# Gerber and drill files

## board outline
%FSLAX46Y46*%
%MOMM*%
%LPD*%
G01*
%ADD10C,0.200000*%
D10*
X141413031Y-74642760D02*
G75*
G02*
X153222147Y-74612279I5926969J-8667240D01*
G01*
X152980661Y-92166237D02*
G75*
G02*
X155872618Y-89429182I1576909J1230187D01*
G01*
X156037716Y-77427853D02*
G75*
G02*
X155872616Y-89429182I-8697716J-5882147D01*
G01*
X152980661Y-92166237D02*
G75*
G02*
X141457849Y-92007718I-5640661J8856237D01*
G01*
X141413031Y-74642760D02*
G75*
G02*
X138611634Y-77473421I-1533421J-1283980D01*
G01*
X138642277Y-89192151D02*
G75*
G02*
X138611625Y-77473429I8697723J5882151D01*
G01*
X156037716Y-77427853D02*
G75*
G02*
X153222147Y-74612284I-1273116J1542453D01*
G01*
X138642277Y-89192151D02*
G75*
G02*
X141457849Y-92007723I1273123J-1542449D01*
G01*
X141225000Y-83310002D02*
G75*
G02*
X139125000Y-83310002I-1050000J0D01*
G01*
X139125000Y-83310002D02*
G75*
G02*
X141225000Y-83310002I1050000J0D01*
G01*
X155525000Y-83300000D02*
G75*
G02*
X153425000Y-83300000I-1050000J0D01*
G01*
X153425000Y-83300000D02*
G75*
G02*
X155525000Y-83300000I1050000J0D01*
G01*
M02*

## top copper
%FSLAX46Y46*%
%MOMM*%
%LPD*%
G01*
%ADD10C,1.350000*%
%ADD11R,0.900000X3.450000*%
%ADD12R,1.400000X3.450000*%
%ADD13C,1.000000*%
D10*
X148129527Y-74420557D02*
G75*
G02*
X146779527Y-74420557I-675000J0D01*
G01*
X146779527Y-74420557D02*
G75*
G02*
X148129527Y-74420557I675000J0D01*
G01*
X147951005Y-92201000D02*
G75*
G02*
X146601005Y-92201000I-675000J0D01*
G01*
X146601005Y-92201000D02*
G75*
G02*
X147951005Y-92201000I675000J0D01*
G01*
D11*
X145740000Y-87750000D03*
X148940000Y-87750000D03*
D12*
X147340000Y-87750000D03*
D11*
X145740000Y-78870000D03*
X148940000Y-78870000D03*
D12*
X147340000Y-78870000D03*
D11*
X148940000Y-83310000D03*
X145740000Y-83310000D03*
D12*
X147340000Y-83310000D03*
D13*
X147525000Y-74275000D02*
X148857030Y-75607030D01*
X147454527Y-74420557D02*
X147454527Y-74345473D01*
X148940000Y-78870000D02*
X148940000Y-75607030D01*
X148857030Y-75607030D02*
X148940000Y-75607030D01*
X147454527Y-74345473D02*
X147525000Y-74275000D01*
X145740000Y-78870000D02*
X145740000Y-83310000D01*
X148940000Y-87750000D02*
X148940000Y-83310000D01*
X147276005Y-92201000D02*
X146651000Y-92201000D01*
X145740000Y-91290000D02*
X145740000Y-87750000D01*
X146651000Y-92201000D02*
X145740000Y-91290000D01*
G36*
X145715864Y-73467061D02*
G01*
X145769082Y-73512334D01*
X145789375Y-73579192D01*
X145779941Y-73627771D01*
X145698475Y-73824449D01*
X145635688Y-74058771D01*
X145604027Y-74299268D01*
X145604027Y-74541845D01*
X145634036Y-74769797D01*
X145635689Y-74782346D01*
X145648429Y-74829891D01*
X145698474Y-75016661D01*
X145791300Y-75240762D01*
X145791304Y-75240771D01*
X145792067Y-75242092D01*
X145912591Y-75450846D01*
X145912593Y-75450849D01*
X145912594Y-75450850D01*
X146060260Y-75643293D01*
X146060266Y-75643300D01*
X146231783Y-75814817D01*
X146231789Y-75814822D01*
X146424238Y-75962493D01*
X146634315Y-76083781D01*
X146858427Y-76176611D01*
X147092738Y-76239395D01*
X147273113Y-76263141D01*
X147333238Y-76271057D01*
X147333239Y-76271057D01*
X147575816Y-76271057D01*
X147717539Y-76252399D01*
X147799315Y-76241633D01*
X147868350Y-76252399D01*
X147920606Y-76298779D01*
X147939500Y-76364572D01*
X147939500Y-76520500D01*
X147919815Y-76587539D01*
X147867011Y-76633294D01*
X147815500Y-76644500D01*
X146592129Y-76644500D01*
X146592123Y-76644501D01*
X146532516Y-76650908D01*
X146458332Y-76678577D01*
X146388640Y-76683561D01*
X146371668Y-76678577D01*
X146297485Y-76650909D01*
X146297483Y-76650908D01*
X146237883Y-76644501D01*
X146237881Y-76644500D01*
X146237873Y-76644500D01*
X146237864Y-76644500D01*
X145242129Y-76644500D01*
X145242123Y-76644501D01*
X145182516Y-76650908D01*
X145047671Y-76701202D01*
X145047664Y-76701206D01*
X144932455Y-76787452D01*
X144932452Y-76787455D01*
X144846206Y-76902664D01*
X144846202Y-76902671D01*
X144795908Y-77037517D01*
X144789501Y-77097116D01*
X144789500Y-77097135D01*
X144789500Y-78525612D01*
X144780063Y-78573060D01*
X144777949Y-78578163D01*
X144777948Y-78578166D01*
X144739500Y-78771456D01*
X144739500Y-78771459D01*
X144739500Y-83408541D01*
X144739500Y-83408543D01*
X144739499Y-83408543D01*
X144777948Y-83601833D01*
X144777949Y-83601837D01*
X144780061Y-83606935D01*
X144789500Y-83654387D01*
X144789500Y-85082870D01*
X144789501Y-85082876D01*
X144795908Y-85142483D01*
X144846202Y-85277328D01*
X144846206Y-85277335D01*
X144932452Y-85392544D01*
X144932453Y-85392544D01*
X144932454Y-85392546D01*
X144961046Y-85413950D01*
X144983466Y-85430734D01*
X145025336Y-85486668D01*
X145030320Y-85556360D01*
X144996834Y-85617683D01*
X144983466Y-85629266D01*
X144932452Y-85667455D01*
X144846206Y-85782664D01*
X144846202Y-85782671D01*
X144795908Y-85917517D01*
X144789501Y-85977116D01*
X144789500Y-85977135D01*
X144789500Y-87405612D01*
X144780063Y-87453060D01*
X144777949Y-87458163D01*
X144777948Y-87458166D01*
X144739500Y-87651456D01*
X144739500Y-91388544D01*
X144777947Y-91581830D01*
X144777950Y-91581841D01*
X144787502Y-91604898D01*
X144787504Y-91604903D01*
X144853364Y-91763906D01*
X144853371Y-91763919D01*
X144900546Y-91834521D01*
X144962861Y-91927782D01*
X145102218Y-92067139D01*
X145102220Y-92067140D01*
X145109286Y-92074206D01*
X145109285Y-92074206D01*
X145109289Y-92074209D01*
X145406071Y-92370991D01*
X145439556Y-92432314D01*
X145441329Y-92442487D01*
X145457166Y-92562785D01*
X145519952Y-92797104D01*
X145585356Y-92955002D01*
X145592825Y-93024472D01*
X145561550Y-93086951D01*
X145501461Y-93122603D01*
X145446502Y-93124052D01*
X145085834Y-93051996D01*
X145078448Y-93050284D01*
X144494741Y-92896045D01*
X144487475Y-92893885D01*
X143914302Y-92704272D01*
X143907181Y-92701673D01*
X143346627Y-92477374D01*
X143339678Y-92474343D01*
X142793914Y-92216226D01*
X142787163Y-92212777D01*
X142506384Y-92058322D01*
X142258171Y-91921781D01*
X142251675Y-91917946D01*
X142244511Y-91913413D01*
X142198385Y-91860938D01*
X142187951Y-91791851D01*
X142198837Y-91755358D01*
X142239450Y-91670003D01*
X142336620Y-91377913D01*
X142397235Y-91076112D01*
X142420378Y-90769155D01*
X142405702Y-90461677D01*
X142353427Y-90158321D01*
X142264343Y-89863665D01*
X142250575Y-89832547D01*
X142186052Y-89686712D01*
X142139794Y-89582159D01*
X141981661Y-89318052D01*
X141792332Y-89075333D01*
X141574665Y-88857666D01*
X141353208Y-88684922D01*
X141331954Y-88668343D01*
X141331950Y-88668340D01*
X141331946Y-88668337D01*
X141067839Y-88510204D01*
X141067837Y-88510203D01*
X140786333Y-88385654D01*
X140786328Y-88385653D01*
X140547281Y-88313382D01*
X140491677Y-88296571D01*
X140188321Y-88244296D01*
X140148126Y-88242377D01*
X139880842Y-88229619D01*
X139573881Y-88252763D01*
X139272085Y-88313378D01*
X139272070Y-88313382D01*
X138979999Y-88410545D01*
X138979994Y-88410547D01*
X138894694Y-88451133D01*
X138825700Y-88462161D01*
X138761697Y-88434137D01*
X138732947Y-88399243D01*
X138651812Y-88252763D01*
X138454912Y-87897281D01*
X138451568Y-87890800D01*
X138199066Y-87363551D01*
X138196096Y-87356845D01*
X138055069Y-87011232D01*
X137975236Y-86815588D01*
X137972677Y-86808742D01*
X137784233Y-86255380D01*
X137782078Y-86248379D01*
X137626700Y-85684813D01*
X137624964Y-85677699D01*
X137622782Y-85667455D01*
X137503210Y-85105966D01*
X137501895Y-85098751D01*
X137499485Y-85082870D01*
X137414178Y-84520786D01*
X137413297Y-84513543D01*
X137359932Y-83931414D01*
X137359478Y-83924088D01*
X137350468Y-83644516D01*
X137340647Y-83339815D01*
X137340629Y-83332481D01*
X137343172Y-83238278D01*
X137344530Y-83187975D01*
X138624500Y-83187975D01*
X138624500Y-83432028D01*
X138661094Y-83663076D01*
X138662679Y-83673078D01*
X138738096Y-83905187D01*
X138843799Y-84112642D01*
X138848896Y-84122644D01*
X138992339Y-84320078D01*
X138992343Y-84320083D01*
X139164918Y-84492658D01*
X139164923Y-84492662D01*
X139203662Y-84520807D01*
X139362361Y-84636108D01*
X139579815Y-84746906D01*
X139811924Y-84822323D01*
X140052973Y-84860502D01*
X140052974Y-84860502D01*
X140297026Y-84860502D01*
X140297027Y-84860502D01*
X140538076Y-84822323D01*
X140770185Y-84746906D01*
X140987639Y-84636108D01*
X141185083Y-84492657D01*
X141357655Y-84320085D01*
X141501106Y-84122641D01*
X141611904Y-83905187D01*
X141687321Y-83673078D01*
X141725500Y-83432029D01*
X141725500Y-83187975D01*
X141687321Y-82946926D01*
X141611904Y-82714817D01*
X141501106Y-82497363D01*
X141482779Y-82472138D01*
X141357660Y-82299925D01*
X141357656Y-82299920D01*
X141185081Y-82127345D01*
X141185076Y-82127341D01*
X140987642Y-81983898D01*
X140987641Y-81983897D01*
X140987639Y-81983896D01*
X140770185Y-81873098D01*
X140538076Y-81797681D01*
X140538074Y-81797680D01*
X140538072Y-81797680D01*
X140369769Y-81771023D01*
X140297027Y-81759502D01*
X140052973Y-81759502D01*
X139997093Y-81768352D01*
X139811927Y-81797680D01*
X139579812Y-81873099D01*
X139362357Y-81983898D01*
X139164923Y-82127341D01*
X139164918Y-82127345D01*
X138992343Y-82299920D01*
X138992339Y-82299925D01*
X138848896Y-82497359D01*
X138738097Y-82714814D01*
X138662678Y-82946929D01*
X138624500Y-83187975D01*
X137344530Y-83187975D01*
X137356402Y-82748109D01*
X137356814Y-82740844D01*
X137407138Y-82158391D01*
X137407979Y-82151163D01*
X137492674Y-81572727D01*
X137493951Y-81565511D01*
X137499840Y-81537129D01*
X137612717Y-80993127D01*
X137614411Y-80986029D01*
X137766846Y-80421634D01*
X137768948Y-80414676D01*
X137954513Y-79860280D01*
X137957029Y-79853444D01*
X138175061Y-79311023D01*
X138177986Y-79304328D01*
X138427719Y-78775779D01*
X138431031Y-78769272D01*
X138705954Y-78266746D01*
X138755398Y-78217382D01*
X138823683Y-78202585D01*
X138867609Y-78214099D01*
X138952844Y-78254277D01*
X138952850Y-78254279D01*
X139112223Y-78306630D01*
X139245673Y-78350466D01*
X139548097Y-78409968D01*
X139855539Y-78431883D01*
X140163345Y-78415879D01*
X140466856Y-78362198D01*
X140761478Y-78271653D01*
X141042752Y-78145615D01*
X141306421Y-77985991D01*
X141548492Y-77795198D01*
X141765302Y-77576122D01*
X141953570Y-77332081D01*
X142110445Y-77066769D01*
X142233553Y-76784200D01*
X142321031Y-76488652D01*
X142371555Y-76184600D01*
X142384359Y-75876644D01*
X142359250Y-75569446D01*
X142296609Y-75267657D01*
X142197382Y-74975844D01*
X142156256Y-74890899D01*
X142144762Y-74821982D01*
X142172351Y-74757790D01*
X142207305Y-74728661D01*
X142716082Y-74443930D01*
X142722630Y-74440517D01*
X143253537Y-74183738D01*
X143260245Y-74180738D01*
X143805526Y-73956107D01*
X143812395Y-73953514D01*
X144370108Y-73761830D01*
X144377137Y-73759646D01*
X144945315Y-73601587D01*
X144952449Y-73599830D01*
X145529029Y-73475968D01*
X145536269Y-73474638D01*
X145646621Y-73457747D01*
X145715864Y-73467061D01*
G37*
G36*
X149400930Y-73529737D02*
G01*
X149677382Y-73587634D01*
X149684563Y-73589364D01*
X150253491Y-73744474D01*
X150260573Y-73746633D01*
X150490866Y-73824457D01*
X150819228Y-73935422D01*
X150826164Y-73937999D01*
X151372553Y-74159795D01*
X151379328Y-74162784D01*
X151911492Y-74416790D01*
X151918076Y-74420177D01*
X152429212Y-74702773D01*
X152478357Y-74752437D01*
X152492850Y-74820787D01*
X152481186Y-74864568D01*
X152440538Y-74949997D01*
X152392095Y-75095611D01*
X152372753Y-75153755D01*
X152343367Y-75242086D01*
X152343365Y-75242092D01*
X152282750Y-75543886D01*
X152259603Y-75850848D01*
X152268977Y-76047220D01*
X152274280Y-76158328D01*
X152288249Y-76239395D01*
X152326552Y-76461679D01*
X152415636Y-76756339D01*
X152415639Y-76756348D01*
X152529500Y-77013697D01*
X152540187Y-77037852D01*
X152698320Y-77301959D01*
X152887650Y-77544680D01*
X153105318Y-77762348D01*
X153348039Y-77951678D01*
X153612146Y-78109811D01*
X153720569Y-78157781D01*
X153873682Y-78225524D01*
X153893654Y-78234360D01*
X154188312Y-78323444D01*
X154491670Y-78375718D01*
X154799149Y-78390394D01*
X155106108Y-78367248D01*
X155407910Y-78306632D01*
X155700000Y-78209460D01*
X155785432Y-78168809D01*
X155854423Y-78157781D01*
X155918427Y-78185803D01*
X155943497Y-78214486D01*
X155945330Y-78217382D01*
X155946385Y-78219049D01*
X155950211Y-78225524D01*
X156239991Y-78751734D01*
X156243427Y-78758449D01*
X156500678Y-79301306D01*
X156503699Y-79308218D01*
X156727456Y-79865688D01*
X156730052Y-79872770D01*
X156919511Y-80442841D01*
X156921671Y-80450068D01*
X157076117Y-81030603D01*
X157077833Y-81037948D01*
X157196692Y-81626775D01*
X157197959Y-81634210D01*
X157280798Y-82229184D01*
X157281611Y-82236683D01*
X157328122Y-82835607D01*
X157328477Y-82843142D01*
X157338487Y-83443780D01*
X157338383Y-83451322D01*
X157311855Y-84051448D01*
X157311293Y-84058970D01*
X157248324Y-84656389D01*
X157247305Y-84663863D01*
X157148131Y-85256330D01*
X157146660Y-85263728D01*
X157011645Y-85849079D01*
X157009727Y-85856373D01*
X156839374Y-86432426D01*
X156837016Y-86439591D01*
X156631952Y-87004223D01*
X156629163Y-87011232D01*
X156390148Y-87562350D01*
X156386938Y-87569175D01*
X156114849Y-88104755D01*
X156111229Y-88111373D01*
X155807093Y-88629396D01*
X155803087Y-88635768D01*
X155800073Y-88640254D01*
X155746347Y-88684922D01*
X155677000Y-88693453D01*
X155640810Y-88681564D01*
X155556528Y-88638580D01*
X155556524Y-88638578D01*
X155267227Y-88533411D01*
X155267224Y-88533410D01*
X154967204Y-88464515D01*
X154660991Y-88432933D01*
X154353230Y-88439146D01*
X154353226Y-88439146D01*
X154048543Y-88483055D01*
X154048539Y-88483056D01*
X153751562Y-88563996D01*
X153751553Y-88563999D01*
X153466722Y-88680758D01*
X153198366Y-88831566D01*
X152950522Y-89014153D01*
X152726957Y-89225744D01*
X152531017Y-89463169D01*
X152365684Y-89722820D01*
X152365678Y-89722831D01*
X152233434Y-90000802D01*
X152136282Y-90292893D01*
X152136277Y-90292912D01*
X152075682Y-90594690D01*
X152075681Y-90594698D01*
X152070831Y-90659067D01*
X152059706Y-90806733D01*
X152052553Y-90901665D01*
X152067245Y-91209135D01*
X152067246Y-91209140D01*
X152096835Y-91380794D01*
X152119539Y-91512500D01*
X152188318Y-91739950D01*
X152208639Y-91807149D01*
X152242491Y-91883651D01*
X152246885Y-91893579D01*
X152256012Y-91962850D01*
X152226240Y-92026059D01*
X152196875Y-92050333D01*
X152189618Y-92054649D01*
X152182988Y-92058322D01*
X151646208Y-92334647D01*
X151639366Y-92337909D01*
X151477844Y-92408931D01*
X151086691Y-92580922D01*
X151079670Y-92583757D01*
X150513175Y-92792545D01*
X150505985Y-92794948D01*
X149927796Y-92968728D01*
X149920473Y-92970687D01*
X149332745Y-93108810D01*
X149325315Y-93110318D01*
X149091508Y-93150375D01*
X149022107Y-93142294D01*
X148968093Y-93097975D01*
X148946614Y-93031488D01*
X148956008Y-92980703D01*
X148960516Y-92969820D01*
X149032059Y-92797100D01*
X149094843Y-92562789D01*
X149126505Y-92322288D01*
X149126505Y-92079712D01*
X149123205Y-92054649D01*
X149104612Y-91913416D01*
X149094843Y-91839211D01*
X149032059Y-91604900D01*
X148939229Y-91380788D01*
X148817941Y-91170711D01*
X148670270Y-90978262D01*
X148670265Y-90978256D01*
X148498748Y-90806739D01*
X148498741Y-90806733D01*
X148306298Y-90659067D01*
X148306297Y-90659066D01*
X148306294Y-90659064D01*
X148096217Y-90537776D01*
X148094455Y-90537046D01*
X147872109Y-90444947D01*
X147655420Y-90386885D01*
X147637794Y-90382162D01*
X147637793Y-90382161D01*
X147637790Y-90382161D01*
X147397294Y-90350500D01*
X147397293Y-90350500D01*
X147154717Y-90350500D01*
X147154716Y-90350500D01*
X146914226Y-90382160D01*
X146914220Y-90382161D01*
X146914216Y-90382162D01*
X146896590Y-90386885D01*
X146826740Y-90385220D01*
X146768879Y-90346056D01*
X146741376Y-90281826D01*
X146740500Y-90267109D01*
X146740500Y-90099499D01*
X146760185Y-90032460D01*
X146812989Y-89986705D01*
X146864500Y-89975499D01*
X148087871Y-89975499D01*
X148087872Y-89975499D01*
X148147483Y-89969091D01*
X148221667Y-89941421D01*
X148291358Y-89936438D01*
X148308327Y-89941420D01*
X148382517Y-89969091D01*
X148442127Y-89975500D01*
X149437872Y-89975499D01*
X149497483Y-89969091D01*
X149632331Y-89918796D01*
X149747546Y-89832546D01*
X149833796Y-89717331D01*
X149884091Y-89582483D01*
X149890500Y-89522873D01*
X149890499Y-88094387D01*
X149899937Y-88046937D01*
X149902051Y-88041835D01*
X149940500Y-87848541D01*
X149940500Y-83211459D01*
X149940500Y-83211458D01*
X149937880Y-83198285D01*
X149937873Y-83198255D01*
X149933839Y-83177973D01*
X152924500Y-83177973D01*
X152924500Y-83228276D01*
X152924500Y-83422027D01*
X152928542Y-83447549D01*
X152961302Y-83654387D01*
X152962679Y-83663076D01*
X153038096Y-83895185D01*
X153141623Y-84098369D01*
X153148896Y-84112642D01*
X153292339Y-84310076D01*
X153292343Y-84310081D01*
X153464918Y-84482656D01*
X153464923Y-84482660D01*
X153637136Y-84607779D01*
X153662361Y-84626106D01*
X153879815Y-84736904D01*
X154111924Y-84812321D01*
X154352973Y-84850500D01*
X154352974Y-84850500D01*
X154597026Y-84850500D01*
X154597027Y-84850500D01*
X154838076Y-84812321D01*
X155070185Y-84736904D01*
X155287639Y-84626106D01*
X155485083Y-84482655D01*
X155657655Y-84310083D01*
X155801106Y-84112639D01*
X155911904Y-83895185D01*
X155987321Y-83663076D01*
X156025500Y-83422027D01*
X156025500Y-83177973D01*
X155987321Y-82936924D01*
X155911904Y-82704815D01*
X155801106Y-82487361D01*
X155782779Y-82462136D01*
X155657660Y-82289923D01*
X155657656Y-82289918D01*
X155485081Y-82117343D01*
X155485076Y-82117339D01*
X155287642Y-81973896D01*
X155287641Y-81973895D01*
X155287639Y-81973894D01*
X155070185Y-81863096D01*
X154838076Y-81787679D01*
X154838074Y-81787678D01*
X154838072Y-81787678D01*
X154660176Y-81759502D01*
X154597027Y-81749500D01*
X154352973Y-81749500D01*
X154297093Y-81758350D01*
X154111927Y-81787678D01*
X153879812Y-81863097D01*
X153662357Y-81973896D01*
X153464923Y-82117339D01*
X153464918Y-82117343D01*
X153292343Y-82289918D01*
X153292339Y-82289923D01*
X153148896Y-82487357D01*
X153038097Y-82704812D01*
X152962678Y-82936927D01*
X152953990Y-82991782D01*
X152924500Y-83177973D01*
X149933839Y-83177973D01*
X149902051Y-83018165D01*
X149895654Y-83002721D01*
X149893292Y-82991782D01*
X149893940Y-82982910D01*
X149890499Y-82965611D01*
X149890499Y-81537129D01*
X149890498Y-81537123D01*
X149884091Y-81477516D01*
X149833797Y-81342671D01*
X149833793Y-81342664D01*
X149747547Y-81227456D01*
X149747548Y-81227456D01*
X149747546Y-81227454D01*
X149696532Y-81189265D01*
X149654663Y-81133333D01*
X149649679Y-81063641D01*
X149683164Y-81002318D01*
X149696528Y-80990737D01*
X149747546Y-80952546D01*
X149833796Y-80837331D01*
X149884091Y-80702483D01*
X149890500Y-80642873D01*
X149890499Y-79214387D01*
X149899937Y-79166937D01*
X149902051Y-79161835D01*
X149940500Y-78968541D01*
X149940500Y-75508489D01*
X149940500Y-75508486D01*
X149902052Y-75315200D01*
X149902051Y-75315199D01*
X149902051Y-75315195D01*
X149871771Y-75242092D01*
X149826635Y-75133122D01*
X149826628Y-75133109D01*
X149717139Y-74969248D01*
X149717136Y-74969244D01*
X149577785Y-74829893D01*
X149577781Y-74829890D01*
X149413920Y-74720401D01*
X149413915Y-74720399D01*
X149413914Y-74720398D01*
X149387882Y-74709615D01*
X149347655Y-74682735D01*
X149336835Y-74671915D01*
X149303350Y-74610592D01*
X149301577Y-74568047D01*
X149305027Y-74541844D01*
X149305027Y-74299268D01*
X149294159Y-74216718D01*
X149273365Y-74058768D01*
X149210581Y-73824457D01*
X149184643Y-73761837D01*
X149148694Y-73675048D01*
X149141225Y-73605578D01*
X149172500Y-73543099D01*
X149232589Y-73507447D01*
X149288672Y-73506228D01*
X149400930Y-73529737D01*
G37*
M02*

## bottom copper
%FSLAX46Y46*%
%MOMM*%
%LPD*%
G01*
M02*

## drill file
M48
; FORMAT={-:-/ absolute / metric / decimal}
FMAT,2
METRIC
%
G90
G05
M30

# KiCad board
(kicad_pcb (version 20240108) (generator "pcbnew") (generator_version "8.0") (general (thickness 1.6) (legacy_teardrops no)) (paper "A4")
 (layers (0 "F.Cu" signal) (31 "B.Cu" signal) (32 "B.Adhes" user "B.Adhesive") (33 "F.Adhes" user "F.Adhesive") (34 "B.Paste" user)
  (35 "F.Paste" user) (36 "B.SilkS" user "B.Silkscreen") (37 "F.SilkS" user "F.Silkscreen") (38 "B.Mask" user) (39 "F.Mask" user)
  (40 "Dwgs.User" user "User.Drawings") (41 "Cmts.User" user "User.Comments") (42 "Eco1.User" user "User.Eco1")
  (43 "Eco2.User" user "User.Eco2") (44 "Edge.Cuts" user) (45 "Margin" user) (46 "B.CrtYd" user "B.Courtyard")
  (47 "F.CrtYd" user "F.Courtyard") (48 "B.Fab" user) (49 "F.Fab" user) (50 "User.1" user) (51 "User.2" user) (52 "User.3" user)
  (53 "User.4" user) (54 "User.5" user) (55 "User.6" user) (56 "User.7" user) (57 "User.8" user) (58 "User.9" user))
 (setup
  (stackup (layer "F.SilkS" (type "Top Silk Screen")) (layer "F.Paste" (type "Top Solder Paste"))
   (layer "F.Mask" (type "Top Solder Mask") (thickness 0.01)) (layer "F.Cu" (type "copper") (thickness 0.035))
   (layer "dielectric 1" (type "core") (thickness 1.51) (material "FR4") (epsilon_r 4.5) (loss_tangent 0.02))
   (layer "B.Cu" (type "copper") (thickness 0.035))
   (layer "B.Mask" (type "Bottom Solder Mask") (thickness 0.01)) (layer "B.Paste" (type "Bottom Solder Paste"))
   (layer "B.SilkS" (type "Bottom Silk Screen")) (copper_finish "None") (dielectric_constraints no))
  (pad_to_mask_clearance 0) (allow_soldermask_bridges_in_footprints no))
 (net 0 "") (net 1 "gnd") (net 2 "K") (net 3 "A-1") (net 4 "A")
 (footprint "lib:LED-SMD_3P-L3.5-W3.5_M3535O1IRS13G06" (layer "F.Cu") (at 147.34 87.75 0)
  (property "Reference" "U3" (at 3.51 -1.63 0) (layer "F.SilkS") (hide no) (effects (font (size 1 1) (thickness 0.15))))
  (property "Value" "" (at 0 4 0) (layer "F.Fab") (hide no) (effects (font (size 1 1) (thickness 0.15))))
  (pad "1" smd rect (at -1.6 0 0) (size 0.9 3.45) (layers "F.Cu" "F.Paste" "F.Mask") (remove_unused_layers no) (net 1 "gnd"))
  (pad "2" smd rect (at 1.6 0 0) (size 0.9 3.45) (layers "F.Cu" "F.Paste" "F.Mask") (remove_unused_layers no) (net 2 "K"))
  (pad "3" smd rect (at 0 0 0) (size 1.4 3.45) (layers "F.Cu" "F.Paste" "F.Mask") (remove_unused_layers no) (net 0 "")))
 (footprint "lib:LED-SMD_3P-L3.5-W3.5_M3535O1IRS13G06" (layer "F.Cu") (at 147.34 78.87 0)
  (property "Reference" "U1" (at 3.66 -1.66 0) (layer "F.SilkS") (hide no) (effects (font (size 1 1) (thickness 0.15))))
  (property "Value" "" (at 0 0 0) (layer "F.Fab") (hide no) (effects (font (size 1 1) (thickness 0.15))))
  (pad "1" smd rect (at -1.6 0 0) (size 0.9 3.45) (layers "F.Cu" "F.Paste" "F.Mask") (remove_unused_layers no) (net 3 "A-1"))
  (pad "2" smd rect (at 1.6 0 0) (size 0.9 3.45) (layers "F.Cu" "F.Paste" "F.Mask") (remove_unused_layers no) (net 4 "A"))
  (pad "3" smd rect (at 0 0 0) (size 1.4 3.45) (layers "F.Cu" "F.Paste" "F.Mask") (remove_unused_layers no) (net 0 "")))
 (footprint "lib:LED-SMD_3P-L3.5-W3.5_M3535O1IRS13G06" (layer "F.Cu") (at 147.34 83.31 180)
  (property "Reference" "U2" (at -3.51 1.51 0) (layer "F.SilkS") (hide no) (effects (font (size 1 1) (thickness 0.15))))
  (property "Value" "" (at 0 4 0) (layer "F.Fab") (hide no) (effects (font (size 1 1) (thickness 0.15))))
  (pad "1" smd rect (at -1.6 0 180) (size 0.9 3.45) (layers "F.Cu" "F.Paste" "F.Mask") (remove_unused_layers no) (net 2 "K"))
  (pad "2" smd rect (at 1.6 0 180) (size 0.9 3.45) (layers "F.Cu" "F.Paste" "F.Mask") (remove_unused_layers no) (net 3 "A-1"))
  (pad "3" smd rect (at 0 0 180) (size 1.4 3.45) (layers "F.Cu" "F.Paste" "F.Mask") (remove_unused_layers no) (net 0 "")))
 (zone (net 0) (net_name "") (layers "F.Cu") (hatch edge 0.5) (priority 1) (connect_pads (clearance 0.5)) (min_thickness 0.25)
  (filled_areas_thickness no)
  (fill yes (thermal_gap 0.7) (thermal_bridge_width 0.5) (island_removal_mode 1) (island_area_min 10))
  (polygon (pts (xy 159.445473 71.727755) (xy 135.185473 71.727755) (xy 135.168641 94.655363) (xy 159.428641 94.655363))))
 (segment (start 147.525 74.275) (end 148.85703 75.60703) (width 1) (layer "F.Cu") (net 4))
 (segment (start 147.454527 74.420557) (end 147.454527 74.345473) (width 1) (layer "F.Cu") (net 4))
 (segment (start 148.94 78.87) (end 148.94 75.60703) (width 1) (layer "F.Cu") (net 4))
 (segment (start 148.85703 75.60703) (end 148.94 75.60703) (width 1) (layer "F.Cu") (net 4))
 (segment (start 147.454527 74.345473) (end 147.525 74.275) (width 1) (layer "F.Cu") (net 4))
 (segment (start 145.74 78.87) (end 145.74 83.31) (width 1) (layer "F.Cu") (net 3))
 (segment (start 148.94 87.75) (end 148.94 83.31) (width 1) (layer "F.Cu") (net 2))
 (segment (start 147.276005 92.201) (end 146.651 92.201) (width 1) (layer "F.Cu") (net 1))
 (segment (start 145.74 91.29) (end 145.74 87.75) (width 1) (layer "F.Cu") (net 1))
 (segment (start 146.651 92.201) (end 145.74 91.29) (width 1) (layer "F.Cu") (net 1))
 (gr_arc (start 141.413031 74.64276) (mid 147.312897 72.810037) (end 153.222145 74.612282) (stroke (width 0.2) (type default))
  (layer "Edge.Cuts"))
 (gr_arc (start 152.980661 92.166237) (mid 153.182794 89.483469) (end 155.872617 89.429183) (stroke (width 0.2) (type default))
  (layer "Edge.Cuts"))
 (gr_arc (start 156.037716 77.427853) (mid 157.839003 83.454433) (end 155.872617 89.429183) (stroke (width 0.2) (type default))
  (layer "Edge.Cuts"))
 (gr_arc (start 152.980661 92.166237) (mid 147.195564 93.809009) (end 141.457847 92.007721) (stroke (width 0.2) (type default))
  (layer "Edge.Cuts"))
 (gr_arc (start 141.413031 74.64276) (mid 141.30115 77.333592) (end 138.611627 77.47343) (stroke (width 0.2) (type default))
  (layer "Edge.Cuts"))
 (gr_arc (start 138.642277 89.192151) (mid 136.840032 83.337464) (end 138.611627 77.47343) (stroke (width 0.2) (type default))
  (layer "Edge.Cuts"))
 (gr_arc (start 156.037716 77.427853) (mid 153.350405 77.299593) (end 153.222145 74.612282) (stroke (width 0.2) (type default))
  (layer "Edge.Cuts"))
 (gr_arc (start 138.642277 89.192151) (mid 141.329577 89.32042) (end 141.457847 92.007721) (stroke (width 0.2) (type default))
  (layer "Edge.Cuts"))
 (gr_circle (center 147.454527 74.420557) (end 148.704527 74.420557) (stroke (width 0.2) (type solid)) (fill solid) (layer "F.Cu"))
 (gr_circle (center 147.276005 92.201) (end 148.526005 92.201) (stroke (width 0.2) (type solid)) (fill solid) (layer "F.Cu"))
 (gr_circle (center 140.175 83.310002) (end 141.225 83.310002) (stroke (width 0.2) (type default)) (fill none) (layer "Edge.Cuts"))
 (gr_circle (center 154.475 83.3) (end 155.525 83.3) (stroke (width 0.2) (type default)) (fill none) (layer "Edge.Cuts")))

